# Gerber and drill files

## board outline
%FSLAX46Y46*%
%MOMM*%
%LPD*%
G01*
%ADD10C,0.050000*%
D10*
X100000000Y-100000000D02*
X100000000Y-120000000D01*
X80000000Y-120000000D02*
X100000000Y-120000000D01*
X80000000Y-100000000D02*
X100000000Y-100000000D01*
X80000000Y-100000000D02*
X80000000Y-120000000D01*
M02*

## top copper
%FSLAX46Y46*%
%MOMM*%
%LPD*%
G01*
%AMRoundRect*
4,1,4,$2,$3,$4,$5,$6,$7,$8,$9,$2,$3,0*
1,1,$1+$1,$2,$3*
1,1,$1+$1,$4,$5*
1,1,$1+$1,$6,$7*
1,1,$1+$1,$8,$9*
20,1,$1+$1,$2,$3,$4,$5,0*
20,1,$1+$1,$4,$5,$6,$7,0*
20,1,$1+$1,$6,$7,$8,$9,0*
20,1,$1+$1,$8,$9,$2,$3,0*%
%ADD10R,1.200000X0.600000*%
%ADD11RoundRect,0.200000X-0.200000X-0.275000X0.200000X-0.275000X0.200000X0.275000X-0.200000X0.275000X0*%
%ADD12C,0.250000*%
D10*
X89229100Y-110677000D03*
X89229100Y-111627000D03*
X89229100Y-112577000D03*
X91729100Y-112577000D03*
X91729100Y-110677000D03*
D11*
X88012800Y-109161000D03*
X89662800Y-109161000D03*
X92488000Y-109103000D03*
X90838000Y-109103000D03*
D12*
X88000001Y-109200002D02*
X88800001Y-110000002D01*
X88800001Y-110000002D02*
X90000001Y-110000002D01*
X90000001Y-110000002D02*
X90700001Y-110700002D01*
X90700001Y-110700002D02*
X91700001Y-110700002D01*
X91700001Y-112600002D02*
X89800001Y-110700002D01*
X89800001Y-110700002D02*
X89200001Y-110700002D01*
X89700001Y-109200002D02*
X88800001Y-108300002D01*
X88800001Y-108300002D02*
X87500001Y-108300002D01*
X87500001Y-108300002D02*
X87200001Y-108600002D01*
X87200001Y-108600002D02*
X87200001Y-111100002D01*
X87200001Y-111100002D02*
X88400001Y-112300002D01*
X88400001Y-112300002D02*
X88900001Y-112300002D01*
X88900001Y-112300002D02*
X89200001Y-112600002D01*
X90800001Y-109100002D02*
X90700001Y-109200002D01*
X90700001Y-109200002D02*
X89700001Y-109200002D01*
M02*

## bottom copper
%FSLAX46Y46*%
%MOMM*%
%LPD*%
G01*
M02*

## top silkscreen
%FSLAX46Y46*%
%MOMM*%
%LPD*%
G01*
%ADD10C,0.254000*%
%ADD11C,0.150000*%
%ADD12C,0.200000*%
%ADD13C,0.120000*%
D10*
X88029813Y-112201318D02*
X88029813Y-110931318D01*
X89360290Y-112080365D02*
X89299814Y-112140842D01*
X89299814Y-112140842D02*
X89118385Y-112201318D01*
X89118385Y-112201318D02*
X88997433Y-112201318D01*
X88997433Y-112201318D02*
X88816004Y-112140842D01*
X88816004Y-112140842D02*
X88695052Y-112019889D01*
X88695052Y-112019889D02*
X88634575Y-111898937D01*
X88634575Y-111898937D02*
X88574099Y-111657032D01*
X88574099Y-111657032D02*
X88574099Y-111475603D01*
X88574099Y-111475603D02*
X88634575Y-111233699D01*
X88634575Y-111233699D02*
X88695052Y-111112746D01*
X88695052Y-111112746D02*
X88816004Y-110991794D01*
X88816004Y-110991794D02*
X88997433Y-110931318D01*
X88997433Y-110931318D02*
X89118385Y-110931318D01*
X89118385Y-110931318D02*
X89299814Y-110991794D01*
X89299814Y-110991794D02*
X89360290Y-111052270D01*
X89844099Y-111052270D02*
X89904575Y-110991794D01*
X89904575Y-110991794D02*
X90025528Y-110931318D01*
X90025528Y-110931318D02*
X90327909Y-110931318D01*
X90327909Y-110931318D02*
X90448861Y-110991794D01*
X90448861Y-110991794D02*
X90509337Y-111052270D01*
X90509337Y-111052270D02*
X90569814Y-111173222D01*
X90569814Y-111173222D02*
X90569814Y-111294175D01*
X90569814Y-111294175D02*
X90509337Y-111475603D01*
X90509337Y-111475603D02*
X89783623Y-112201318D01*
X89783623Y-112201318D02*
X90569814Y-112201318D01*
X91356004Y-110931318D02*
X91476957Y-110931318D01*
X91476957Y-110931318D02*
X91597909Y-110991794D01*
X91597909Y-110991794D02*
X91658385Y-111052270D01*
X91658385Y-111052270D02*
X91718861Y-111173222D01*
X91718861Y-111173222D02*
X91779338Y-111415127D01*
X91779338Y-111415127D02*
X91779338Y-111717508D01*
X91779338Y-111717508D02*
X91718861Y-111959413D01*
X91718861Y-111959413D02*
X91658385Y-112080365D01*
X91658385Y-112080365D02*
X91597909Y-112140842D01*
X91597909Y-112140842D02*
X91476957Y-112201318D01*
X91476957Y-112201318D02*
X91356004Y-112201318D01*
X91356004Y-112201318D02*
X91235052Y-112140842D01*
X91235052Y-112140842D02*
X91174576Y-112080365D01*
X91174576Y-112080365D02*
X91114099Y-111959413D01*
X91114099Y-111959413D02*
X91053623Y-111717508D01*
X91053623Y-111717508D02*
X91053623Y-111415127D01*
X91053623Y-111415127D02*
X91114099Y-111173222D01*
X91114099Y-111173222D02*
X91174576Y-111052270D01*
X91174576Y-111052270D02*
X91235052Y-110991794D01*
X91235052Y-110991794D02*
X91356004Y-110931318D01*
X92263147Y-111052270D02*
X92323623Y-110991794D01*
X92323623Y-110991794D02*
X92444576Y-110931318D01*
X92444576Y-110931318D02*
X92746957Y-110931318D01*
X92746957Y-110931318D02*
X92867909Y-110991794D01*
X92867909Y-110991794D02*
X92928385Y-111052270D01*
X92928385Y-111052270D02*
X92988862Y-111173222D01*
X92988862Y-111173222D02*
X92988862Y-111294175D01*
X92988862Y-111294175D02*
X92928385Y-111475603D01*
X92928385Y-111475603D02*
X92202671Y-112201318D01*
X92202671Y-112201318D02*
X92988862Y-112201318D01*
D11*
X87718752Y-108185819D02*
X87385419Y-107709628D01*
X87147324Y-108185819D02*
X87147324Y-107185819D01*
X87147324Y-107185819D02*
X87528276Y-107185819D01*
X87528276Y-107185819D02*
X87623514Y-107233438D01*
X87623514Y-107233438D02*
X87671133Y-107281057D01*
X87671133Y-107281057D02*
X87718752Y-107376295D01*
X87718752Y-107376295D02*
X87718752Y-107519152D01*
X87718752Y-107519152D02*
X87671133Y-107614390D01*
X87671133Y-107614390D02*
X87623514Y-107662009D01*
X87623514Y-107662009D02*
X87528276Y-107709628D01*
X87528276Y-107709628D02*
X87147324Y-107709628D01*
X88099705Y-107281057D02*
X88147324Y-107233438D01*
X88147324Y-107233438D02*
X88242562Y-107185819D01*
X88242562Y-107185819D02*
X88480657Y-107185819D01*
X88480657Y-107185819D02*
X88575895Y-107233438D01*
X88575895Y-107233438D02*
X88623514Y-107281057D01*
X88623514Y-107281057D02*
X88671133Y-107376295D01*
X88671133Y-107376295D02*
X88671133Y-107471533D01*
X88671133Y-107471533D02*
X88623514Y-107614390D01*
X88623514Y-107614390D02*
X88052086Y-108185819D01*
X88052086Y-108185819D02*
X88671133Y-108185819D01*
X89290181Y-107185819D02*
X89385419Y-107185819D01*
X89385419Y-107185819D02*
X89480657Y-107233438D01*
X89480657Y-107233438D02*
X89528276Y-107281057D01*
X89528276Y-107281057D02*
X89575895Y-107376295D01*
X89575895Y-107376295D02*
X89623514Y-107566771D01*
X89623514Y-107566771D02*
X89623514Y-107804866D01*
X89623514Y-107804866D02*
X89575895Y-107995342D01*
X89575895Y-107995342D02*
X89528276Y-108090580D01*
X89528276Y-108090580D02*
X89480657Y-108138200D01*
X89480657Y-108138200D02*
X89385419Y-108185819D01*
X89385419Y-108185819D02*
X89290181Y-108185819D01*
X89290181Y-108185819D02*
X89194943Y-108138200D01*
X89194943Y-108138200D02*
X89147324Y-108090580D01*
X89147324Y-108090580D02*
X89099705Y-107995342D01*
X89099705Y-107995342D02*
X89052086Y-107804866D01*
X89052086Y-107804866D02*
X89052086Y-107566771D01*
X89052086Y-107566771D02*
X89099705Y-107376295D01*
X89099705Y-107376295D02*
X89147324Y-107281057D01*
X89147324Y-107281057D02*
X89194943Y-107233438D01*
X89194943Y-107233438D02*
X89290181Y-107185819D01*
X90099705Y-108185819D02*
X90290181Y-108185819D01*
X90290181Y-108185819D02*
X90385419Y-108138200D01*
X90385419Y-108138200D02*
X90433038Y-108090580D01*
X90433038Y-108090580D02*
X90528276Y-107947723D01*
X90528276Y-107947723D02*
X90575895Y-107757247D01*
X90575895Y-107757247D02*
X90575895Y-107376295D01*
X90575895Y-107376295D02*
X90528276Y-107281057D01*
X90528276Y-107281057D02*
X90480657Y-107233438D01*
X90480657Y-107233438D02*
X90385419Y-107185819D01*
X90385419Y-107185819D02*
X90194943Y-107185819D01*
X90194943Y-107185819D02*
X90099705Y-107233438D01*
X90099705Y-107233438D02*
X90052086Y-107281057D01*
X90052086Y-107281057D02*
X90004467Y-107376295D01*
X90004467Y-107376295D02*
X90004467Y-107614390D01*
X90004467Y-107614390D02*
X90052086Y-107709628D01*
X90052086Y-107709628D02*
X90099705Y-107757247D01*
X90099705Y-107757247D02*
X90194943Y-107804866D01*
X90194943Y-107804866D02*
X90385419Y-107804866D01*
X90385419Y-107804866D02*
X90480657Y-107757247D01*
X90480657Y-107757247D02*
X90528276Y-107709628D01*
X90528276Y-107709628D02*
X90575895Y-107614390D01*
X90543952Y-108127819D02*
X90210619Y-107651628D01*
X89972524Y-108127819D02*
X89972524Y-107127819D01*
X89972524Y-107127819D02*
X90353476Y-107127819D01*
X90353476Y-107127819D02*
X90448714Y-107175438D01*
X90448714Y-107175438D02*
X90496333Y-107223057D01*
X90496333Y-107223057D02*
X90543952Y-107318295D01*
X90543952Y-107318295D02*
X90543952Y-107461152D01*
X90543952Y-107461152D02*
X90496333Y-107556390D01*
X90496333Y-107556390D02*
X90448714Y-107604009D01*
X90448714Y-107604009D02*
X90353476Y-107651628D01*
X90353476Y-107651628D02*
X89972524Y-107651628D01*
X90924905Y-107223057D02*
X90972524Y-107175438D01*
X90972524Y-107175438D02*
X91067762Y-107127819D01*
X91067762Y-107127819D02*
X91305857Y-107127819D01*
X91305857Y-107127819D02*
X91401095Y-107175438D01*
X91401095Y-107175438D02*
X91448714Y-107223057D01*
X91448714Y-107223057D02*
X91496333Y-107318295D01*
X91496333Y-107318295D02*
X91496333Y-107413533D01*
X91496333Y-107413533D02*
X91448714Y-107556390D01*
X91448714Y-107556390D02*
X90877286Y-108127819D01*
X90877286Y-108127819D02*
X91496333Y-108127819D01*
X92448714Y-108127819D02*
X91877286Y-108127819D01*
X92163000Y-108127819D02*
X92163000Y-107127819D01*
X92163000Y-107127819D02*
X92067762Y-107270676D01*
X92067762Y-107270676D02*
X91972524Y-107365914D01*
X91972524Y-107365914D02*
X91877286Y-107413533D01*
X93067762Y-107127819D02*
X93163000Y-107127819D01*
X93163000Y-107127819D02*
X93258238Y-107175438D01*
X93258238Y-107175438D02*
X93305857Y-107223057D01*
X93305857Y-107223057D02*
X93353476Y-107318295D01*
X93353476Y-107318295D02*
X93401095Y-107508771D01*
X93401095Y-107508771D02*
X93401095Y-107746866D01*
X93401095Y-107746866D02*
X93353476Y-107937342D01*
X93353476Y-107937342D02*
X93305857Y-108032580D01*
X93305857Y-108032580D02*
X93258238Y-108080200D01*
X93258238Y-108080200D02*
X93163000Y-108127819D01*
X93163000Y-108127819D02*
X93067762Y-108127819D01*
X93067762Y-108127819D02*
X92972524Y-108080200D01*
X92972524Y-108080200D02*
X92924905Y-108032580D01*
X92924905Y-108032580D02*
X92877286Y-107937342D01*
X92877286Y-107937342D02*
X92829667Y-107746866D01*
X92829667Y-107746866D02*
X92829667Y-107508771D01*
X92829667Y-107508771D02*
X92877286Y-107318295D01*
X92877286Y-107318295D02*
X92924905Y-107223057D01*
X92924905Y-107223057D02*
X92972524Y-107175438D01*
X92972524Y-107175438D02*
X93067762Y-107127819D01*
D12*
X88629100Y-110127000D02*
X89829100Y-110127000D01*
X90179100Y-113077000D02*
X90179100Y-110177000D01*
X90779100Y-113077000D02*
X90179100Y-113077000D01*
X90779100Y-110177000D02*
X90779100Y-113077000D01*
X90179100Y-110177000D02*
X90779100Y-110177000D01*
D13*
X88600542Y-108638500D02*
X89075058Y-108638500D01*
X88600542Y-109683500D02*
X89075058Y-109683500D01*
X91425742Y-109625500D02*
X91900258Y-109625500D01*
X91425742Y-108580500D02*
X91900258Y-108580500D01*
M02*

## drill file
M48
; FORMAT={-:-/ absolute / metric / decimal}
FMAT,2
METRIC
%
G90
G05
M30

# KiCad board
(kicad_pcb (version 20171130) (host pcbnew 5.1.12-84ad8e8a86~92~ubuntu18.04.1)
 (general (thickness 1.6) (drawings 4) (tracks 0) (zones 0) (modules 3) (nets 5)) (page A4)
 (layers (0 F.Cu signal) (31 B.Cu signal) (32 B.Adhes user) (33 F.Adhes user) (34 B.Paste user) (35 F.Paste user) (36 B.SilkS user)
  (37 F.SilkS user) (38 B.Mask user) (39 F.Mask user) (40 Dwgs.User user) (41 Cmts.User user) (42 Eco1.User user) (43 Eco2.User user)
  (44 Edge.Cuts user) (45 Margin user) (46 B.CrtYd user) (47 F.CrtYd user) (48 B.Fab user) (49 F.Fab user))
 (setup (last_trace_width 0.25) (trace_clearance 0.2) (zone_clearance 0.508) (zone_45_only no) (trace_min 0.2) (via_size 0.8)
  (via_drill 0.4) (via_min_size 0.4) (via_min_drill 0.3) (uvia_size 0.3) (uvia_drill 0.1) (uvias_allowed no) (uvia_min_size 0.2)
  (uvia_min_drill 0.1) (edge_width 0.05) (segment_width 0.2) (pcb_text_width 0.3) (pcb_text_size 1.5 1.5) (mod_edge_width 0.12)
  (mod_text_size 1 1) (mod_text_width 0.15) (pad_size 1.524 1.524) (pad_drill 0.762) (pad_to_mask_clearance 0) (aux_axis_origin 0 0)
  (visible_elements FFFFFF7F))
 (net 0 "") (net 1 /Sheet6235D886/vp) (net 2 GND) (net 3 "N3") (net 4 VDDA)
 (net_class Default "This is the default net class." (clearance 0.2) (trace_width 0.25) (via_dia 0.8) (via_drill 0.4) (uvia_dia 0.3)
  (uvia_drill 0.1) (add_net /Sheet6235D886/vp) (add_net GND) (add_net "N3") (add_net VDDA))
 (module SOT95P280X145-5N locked (layer F.Cu) (at 90.479100 111.627000)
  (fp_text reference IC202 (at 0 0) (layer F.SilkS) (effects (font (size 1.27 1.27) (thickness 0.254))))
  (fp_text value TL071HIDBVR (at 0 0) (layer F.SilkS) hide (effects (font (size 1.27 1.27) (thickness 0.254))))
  (fp_line (start -1.85 -1.5) (end -0.65 -1.5) (layer F.SilkS) (width 0.2))
  (fp_line (start -0.3 1.45) (end -0.3 -1.45) (layer F.SilkS) (width 0.2))
  (fp_line (start 0.3 1.45) (end -0.3 1.45) (layer F.SilkS) (width 0.2))
  (fp_line (start 0.3 -1.45) (end 0.3 1.45) (layer F.SilkS) (width 0.2))
  (fp_line (start -0.3 -1.45) (end 0.3 -1.45) (layer F.SilkS) (width 0.2))
  (pad 1 smd rect (at -1.25 -0.95 90.000000) (size 0.6 1.2) (layers F.Cu F.Mask F.Paste) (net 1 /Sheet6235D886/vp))
  (pad 2 smd rect (at -1.25 0 90.000000) (size 0.6 1.2) (layers F.Cu F.Mask F.Paste) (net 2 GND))
  (pad 3 smd rect (at -1.25 0.95 90.000000) (size 0.6 1.2) (layers F.Cu F.Mask F.Paste) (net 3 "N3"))
  (pad 4 smd rect (at 1.25 0.95 90.000000) (size 0.6 1.2) (layers F.Cu F.Mask F.Paste) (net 1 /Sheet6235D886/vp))
  (pad 5 smd rect (at 1.25 -0.95 90.000000) (size 0.6 1.2) (layers F.Cu F.Mask F.Paste) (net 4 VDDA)))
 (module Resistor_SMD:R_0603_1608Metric (layer F.Cu) (at 88.837800 109.161000)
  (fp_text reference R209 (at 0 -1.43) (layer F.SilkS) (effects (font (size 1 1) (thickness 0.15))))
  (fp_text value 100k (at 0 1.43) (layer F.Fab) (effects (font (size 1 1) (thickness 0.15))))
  (fp_line (start -0.237258 -0.5225) (end 0.237258 -0.5225) (layer F.SilkS) (width 0.12))
  (fp_line (start -0.237258 0.5225) (end 0.237258 0.5225) (layer F.SilkS) (width 0.12))
  (pad 1 smd roundrect (at -0.825 0) (size 0.8 0.95) (layers F.Cu F.Mask F.Paste) (roundrect_rratio 0.25) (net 4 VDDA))
  (pad 2 smd roundrect (at 0.825 0) (size 0.8 0.95) (layers F.Cu F.Mask F.Paste) (roundrect_rratio 0.25) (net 3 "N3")))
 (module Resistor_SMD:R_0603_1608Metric (layer F.Cu) (at 91.663000 109.103000)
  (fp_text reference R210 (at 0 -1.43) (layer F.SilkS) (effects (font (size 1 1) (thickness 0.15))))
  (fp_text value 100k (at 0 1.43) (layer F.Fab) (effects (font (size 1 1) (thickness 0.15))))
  (fp_line (start -0.237258 0.5225) (end 0.237258 0.5225) (layer F.SilkS) (width 0.12))
  (fp_line (start -0.237258 -0.5225) (end 0.237258 -0.5225) (layer F.SilkS) (width 0.12))
  (pad 2 smd roundrect (at 0.825 0) (size 0.8 0.95) (layers F.Cu F.Mask F.Paste) (roundrect_rratio 0.25) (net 2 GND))
  (pad 1 smd roundrect (at -0.825 0) (size 0.8 0.95) (layers F.Cu F.Mask F.Paste) (roundrect_rratio 0.25) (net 3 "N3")))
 (gr_line (start 100 100) (end 100 120) (layer Edge.Cuts) (width 0.05))
 (gr_line (start 80 120) (end 100 120) (layer Edge.Cuts) (width 0.05))
 (gr_line (start 80 100) (end 100 100) (layer Edge.Cuts) (width 0.05))
 (gr_line (start 80 100) (end 80 120) (layer Edge.Cuts) (width 0.05))
 (segment (start 88.000001 109.200002) (end 88.800001 110.000002) (width 0.250000) (layer F.Cu) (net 4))
 (segment (start 88.800001 110.000002) (end 90.000001 110.000002) (width 0.250000) (layer F.Cu) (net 4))
 (segment (start 90.000001 110.000002) (end 90.700001 110.700002) (width 0.250000) (layer F.Cu) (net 4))
 (segment (start 90.700001 110.700002) (end 91.700001 110.700002) (width 0.250000) (layer F.Cu) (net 4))
 (segment (start 91.700001 112.600002) (end 89.800001 110.700002) (width 0.250000) (layer F.Cu) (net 1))
 (segment (start 89.800001 110.700002) (end 89.200001 110.700002) (width 0.250000) (layer F.Cu) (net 1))
 (segment (start 89.700001 109.200002) (end 88.800001 108.300002) (width 0.250000) (layer F.Cu) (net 3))
 (segment (start 88.800001 108.300002) (end 87.500001 108.300002) (width 0.250000) (layer F.Cu) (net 3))
 (segment (start 87.500001 108.300002) (end 87.200001 108.600002) (width 0.250000) (layer F.Cu) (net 3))
 (segment (start 87.200001 108.600002) (end 87.200001 111.100002) (width 0.250000) (layer F.Cu) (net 3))
 (segment (start 87.200001 111.100002) (end 88.400001 112.300002) (width 0.250000) (layer F.Cu) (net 3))
 (segment (start 88.400001 112.300002) (end 88.900001 112.300002) (width 0.250000) (layer F.Cu) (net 3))
 (segment (start 88.900001 112.300002) (end 89.200001 112.600002) (width 0.250000) (layer F.Cu) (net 3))
 (segment (start 90.800001 109.100002) (end 90.700001 109.200002) (width 0.250000) (layer F.Cu) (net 3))
 (segment (start 90.700001 109.200002) (end 89.700001 109.200002) (width 0.250000) (layer F.Cu) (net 3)))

